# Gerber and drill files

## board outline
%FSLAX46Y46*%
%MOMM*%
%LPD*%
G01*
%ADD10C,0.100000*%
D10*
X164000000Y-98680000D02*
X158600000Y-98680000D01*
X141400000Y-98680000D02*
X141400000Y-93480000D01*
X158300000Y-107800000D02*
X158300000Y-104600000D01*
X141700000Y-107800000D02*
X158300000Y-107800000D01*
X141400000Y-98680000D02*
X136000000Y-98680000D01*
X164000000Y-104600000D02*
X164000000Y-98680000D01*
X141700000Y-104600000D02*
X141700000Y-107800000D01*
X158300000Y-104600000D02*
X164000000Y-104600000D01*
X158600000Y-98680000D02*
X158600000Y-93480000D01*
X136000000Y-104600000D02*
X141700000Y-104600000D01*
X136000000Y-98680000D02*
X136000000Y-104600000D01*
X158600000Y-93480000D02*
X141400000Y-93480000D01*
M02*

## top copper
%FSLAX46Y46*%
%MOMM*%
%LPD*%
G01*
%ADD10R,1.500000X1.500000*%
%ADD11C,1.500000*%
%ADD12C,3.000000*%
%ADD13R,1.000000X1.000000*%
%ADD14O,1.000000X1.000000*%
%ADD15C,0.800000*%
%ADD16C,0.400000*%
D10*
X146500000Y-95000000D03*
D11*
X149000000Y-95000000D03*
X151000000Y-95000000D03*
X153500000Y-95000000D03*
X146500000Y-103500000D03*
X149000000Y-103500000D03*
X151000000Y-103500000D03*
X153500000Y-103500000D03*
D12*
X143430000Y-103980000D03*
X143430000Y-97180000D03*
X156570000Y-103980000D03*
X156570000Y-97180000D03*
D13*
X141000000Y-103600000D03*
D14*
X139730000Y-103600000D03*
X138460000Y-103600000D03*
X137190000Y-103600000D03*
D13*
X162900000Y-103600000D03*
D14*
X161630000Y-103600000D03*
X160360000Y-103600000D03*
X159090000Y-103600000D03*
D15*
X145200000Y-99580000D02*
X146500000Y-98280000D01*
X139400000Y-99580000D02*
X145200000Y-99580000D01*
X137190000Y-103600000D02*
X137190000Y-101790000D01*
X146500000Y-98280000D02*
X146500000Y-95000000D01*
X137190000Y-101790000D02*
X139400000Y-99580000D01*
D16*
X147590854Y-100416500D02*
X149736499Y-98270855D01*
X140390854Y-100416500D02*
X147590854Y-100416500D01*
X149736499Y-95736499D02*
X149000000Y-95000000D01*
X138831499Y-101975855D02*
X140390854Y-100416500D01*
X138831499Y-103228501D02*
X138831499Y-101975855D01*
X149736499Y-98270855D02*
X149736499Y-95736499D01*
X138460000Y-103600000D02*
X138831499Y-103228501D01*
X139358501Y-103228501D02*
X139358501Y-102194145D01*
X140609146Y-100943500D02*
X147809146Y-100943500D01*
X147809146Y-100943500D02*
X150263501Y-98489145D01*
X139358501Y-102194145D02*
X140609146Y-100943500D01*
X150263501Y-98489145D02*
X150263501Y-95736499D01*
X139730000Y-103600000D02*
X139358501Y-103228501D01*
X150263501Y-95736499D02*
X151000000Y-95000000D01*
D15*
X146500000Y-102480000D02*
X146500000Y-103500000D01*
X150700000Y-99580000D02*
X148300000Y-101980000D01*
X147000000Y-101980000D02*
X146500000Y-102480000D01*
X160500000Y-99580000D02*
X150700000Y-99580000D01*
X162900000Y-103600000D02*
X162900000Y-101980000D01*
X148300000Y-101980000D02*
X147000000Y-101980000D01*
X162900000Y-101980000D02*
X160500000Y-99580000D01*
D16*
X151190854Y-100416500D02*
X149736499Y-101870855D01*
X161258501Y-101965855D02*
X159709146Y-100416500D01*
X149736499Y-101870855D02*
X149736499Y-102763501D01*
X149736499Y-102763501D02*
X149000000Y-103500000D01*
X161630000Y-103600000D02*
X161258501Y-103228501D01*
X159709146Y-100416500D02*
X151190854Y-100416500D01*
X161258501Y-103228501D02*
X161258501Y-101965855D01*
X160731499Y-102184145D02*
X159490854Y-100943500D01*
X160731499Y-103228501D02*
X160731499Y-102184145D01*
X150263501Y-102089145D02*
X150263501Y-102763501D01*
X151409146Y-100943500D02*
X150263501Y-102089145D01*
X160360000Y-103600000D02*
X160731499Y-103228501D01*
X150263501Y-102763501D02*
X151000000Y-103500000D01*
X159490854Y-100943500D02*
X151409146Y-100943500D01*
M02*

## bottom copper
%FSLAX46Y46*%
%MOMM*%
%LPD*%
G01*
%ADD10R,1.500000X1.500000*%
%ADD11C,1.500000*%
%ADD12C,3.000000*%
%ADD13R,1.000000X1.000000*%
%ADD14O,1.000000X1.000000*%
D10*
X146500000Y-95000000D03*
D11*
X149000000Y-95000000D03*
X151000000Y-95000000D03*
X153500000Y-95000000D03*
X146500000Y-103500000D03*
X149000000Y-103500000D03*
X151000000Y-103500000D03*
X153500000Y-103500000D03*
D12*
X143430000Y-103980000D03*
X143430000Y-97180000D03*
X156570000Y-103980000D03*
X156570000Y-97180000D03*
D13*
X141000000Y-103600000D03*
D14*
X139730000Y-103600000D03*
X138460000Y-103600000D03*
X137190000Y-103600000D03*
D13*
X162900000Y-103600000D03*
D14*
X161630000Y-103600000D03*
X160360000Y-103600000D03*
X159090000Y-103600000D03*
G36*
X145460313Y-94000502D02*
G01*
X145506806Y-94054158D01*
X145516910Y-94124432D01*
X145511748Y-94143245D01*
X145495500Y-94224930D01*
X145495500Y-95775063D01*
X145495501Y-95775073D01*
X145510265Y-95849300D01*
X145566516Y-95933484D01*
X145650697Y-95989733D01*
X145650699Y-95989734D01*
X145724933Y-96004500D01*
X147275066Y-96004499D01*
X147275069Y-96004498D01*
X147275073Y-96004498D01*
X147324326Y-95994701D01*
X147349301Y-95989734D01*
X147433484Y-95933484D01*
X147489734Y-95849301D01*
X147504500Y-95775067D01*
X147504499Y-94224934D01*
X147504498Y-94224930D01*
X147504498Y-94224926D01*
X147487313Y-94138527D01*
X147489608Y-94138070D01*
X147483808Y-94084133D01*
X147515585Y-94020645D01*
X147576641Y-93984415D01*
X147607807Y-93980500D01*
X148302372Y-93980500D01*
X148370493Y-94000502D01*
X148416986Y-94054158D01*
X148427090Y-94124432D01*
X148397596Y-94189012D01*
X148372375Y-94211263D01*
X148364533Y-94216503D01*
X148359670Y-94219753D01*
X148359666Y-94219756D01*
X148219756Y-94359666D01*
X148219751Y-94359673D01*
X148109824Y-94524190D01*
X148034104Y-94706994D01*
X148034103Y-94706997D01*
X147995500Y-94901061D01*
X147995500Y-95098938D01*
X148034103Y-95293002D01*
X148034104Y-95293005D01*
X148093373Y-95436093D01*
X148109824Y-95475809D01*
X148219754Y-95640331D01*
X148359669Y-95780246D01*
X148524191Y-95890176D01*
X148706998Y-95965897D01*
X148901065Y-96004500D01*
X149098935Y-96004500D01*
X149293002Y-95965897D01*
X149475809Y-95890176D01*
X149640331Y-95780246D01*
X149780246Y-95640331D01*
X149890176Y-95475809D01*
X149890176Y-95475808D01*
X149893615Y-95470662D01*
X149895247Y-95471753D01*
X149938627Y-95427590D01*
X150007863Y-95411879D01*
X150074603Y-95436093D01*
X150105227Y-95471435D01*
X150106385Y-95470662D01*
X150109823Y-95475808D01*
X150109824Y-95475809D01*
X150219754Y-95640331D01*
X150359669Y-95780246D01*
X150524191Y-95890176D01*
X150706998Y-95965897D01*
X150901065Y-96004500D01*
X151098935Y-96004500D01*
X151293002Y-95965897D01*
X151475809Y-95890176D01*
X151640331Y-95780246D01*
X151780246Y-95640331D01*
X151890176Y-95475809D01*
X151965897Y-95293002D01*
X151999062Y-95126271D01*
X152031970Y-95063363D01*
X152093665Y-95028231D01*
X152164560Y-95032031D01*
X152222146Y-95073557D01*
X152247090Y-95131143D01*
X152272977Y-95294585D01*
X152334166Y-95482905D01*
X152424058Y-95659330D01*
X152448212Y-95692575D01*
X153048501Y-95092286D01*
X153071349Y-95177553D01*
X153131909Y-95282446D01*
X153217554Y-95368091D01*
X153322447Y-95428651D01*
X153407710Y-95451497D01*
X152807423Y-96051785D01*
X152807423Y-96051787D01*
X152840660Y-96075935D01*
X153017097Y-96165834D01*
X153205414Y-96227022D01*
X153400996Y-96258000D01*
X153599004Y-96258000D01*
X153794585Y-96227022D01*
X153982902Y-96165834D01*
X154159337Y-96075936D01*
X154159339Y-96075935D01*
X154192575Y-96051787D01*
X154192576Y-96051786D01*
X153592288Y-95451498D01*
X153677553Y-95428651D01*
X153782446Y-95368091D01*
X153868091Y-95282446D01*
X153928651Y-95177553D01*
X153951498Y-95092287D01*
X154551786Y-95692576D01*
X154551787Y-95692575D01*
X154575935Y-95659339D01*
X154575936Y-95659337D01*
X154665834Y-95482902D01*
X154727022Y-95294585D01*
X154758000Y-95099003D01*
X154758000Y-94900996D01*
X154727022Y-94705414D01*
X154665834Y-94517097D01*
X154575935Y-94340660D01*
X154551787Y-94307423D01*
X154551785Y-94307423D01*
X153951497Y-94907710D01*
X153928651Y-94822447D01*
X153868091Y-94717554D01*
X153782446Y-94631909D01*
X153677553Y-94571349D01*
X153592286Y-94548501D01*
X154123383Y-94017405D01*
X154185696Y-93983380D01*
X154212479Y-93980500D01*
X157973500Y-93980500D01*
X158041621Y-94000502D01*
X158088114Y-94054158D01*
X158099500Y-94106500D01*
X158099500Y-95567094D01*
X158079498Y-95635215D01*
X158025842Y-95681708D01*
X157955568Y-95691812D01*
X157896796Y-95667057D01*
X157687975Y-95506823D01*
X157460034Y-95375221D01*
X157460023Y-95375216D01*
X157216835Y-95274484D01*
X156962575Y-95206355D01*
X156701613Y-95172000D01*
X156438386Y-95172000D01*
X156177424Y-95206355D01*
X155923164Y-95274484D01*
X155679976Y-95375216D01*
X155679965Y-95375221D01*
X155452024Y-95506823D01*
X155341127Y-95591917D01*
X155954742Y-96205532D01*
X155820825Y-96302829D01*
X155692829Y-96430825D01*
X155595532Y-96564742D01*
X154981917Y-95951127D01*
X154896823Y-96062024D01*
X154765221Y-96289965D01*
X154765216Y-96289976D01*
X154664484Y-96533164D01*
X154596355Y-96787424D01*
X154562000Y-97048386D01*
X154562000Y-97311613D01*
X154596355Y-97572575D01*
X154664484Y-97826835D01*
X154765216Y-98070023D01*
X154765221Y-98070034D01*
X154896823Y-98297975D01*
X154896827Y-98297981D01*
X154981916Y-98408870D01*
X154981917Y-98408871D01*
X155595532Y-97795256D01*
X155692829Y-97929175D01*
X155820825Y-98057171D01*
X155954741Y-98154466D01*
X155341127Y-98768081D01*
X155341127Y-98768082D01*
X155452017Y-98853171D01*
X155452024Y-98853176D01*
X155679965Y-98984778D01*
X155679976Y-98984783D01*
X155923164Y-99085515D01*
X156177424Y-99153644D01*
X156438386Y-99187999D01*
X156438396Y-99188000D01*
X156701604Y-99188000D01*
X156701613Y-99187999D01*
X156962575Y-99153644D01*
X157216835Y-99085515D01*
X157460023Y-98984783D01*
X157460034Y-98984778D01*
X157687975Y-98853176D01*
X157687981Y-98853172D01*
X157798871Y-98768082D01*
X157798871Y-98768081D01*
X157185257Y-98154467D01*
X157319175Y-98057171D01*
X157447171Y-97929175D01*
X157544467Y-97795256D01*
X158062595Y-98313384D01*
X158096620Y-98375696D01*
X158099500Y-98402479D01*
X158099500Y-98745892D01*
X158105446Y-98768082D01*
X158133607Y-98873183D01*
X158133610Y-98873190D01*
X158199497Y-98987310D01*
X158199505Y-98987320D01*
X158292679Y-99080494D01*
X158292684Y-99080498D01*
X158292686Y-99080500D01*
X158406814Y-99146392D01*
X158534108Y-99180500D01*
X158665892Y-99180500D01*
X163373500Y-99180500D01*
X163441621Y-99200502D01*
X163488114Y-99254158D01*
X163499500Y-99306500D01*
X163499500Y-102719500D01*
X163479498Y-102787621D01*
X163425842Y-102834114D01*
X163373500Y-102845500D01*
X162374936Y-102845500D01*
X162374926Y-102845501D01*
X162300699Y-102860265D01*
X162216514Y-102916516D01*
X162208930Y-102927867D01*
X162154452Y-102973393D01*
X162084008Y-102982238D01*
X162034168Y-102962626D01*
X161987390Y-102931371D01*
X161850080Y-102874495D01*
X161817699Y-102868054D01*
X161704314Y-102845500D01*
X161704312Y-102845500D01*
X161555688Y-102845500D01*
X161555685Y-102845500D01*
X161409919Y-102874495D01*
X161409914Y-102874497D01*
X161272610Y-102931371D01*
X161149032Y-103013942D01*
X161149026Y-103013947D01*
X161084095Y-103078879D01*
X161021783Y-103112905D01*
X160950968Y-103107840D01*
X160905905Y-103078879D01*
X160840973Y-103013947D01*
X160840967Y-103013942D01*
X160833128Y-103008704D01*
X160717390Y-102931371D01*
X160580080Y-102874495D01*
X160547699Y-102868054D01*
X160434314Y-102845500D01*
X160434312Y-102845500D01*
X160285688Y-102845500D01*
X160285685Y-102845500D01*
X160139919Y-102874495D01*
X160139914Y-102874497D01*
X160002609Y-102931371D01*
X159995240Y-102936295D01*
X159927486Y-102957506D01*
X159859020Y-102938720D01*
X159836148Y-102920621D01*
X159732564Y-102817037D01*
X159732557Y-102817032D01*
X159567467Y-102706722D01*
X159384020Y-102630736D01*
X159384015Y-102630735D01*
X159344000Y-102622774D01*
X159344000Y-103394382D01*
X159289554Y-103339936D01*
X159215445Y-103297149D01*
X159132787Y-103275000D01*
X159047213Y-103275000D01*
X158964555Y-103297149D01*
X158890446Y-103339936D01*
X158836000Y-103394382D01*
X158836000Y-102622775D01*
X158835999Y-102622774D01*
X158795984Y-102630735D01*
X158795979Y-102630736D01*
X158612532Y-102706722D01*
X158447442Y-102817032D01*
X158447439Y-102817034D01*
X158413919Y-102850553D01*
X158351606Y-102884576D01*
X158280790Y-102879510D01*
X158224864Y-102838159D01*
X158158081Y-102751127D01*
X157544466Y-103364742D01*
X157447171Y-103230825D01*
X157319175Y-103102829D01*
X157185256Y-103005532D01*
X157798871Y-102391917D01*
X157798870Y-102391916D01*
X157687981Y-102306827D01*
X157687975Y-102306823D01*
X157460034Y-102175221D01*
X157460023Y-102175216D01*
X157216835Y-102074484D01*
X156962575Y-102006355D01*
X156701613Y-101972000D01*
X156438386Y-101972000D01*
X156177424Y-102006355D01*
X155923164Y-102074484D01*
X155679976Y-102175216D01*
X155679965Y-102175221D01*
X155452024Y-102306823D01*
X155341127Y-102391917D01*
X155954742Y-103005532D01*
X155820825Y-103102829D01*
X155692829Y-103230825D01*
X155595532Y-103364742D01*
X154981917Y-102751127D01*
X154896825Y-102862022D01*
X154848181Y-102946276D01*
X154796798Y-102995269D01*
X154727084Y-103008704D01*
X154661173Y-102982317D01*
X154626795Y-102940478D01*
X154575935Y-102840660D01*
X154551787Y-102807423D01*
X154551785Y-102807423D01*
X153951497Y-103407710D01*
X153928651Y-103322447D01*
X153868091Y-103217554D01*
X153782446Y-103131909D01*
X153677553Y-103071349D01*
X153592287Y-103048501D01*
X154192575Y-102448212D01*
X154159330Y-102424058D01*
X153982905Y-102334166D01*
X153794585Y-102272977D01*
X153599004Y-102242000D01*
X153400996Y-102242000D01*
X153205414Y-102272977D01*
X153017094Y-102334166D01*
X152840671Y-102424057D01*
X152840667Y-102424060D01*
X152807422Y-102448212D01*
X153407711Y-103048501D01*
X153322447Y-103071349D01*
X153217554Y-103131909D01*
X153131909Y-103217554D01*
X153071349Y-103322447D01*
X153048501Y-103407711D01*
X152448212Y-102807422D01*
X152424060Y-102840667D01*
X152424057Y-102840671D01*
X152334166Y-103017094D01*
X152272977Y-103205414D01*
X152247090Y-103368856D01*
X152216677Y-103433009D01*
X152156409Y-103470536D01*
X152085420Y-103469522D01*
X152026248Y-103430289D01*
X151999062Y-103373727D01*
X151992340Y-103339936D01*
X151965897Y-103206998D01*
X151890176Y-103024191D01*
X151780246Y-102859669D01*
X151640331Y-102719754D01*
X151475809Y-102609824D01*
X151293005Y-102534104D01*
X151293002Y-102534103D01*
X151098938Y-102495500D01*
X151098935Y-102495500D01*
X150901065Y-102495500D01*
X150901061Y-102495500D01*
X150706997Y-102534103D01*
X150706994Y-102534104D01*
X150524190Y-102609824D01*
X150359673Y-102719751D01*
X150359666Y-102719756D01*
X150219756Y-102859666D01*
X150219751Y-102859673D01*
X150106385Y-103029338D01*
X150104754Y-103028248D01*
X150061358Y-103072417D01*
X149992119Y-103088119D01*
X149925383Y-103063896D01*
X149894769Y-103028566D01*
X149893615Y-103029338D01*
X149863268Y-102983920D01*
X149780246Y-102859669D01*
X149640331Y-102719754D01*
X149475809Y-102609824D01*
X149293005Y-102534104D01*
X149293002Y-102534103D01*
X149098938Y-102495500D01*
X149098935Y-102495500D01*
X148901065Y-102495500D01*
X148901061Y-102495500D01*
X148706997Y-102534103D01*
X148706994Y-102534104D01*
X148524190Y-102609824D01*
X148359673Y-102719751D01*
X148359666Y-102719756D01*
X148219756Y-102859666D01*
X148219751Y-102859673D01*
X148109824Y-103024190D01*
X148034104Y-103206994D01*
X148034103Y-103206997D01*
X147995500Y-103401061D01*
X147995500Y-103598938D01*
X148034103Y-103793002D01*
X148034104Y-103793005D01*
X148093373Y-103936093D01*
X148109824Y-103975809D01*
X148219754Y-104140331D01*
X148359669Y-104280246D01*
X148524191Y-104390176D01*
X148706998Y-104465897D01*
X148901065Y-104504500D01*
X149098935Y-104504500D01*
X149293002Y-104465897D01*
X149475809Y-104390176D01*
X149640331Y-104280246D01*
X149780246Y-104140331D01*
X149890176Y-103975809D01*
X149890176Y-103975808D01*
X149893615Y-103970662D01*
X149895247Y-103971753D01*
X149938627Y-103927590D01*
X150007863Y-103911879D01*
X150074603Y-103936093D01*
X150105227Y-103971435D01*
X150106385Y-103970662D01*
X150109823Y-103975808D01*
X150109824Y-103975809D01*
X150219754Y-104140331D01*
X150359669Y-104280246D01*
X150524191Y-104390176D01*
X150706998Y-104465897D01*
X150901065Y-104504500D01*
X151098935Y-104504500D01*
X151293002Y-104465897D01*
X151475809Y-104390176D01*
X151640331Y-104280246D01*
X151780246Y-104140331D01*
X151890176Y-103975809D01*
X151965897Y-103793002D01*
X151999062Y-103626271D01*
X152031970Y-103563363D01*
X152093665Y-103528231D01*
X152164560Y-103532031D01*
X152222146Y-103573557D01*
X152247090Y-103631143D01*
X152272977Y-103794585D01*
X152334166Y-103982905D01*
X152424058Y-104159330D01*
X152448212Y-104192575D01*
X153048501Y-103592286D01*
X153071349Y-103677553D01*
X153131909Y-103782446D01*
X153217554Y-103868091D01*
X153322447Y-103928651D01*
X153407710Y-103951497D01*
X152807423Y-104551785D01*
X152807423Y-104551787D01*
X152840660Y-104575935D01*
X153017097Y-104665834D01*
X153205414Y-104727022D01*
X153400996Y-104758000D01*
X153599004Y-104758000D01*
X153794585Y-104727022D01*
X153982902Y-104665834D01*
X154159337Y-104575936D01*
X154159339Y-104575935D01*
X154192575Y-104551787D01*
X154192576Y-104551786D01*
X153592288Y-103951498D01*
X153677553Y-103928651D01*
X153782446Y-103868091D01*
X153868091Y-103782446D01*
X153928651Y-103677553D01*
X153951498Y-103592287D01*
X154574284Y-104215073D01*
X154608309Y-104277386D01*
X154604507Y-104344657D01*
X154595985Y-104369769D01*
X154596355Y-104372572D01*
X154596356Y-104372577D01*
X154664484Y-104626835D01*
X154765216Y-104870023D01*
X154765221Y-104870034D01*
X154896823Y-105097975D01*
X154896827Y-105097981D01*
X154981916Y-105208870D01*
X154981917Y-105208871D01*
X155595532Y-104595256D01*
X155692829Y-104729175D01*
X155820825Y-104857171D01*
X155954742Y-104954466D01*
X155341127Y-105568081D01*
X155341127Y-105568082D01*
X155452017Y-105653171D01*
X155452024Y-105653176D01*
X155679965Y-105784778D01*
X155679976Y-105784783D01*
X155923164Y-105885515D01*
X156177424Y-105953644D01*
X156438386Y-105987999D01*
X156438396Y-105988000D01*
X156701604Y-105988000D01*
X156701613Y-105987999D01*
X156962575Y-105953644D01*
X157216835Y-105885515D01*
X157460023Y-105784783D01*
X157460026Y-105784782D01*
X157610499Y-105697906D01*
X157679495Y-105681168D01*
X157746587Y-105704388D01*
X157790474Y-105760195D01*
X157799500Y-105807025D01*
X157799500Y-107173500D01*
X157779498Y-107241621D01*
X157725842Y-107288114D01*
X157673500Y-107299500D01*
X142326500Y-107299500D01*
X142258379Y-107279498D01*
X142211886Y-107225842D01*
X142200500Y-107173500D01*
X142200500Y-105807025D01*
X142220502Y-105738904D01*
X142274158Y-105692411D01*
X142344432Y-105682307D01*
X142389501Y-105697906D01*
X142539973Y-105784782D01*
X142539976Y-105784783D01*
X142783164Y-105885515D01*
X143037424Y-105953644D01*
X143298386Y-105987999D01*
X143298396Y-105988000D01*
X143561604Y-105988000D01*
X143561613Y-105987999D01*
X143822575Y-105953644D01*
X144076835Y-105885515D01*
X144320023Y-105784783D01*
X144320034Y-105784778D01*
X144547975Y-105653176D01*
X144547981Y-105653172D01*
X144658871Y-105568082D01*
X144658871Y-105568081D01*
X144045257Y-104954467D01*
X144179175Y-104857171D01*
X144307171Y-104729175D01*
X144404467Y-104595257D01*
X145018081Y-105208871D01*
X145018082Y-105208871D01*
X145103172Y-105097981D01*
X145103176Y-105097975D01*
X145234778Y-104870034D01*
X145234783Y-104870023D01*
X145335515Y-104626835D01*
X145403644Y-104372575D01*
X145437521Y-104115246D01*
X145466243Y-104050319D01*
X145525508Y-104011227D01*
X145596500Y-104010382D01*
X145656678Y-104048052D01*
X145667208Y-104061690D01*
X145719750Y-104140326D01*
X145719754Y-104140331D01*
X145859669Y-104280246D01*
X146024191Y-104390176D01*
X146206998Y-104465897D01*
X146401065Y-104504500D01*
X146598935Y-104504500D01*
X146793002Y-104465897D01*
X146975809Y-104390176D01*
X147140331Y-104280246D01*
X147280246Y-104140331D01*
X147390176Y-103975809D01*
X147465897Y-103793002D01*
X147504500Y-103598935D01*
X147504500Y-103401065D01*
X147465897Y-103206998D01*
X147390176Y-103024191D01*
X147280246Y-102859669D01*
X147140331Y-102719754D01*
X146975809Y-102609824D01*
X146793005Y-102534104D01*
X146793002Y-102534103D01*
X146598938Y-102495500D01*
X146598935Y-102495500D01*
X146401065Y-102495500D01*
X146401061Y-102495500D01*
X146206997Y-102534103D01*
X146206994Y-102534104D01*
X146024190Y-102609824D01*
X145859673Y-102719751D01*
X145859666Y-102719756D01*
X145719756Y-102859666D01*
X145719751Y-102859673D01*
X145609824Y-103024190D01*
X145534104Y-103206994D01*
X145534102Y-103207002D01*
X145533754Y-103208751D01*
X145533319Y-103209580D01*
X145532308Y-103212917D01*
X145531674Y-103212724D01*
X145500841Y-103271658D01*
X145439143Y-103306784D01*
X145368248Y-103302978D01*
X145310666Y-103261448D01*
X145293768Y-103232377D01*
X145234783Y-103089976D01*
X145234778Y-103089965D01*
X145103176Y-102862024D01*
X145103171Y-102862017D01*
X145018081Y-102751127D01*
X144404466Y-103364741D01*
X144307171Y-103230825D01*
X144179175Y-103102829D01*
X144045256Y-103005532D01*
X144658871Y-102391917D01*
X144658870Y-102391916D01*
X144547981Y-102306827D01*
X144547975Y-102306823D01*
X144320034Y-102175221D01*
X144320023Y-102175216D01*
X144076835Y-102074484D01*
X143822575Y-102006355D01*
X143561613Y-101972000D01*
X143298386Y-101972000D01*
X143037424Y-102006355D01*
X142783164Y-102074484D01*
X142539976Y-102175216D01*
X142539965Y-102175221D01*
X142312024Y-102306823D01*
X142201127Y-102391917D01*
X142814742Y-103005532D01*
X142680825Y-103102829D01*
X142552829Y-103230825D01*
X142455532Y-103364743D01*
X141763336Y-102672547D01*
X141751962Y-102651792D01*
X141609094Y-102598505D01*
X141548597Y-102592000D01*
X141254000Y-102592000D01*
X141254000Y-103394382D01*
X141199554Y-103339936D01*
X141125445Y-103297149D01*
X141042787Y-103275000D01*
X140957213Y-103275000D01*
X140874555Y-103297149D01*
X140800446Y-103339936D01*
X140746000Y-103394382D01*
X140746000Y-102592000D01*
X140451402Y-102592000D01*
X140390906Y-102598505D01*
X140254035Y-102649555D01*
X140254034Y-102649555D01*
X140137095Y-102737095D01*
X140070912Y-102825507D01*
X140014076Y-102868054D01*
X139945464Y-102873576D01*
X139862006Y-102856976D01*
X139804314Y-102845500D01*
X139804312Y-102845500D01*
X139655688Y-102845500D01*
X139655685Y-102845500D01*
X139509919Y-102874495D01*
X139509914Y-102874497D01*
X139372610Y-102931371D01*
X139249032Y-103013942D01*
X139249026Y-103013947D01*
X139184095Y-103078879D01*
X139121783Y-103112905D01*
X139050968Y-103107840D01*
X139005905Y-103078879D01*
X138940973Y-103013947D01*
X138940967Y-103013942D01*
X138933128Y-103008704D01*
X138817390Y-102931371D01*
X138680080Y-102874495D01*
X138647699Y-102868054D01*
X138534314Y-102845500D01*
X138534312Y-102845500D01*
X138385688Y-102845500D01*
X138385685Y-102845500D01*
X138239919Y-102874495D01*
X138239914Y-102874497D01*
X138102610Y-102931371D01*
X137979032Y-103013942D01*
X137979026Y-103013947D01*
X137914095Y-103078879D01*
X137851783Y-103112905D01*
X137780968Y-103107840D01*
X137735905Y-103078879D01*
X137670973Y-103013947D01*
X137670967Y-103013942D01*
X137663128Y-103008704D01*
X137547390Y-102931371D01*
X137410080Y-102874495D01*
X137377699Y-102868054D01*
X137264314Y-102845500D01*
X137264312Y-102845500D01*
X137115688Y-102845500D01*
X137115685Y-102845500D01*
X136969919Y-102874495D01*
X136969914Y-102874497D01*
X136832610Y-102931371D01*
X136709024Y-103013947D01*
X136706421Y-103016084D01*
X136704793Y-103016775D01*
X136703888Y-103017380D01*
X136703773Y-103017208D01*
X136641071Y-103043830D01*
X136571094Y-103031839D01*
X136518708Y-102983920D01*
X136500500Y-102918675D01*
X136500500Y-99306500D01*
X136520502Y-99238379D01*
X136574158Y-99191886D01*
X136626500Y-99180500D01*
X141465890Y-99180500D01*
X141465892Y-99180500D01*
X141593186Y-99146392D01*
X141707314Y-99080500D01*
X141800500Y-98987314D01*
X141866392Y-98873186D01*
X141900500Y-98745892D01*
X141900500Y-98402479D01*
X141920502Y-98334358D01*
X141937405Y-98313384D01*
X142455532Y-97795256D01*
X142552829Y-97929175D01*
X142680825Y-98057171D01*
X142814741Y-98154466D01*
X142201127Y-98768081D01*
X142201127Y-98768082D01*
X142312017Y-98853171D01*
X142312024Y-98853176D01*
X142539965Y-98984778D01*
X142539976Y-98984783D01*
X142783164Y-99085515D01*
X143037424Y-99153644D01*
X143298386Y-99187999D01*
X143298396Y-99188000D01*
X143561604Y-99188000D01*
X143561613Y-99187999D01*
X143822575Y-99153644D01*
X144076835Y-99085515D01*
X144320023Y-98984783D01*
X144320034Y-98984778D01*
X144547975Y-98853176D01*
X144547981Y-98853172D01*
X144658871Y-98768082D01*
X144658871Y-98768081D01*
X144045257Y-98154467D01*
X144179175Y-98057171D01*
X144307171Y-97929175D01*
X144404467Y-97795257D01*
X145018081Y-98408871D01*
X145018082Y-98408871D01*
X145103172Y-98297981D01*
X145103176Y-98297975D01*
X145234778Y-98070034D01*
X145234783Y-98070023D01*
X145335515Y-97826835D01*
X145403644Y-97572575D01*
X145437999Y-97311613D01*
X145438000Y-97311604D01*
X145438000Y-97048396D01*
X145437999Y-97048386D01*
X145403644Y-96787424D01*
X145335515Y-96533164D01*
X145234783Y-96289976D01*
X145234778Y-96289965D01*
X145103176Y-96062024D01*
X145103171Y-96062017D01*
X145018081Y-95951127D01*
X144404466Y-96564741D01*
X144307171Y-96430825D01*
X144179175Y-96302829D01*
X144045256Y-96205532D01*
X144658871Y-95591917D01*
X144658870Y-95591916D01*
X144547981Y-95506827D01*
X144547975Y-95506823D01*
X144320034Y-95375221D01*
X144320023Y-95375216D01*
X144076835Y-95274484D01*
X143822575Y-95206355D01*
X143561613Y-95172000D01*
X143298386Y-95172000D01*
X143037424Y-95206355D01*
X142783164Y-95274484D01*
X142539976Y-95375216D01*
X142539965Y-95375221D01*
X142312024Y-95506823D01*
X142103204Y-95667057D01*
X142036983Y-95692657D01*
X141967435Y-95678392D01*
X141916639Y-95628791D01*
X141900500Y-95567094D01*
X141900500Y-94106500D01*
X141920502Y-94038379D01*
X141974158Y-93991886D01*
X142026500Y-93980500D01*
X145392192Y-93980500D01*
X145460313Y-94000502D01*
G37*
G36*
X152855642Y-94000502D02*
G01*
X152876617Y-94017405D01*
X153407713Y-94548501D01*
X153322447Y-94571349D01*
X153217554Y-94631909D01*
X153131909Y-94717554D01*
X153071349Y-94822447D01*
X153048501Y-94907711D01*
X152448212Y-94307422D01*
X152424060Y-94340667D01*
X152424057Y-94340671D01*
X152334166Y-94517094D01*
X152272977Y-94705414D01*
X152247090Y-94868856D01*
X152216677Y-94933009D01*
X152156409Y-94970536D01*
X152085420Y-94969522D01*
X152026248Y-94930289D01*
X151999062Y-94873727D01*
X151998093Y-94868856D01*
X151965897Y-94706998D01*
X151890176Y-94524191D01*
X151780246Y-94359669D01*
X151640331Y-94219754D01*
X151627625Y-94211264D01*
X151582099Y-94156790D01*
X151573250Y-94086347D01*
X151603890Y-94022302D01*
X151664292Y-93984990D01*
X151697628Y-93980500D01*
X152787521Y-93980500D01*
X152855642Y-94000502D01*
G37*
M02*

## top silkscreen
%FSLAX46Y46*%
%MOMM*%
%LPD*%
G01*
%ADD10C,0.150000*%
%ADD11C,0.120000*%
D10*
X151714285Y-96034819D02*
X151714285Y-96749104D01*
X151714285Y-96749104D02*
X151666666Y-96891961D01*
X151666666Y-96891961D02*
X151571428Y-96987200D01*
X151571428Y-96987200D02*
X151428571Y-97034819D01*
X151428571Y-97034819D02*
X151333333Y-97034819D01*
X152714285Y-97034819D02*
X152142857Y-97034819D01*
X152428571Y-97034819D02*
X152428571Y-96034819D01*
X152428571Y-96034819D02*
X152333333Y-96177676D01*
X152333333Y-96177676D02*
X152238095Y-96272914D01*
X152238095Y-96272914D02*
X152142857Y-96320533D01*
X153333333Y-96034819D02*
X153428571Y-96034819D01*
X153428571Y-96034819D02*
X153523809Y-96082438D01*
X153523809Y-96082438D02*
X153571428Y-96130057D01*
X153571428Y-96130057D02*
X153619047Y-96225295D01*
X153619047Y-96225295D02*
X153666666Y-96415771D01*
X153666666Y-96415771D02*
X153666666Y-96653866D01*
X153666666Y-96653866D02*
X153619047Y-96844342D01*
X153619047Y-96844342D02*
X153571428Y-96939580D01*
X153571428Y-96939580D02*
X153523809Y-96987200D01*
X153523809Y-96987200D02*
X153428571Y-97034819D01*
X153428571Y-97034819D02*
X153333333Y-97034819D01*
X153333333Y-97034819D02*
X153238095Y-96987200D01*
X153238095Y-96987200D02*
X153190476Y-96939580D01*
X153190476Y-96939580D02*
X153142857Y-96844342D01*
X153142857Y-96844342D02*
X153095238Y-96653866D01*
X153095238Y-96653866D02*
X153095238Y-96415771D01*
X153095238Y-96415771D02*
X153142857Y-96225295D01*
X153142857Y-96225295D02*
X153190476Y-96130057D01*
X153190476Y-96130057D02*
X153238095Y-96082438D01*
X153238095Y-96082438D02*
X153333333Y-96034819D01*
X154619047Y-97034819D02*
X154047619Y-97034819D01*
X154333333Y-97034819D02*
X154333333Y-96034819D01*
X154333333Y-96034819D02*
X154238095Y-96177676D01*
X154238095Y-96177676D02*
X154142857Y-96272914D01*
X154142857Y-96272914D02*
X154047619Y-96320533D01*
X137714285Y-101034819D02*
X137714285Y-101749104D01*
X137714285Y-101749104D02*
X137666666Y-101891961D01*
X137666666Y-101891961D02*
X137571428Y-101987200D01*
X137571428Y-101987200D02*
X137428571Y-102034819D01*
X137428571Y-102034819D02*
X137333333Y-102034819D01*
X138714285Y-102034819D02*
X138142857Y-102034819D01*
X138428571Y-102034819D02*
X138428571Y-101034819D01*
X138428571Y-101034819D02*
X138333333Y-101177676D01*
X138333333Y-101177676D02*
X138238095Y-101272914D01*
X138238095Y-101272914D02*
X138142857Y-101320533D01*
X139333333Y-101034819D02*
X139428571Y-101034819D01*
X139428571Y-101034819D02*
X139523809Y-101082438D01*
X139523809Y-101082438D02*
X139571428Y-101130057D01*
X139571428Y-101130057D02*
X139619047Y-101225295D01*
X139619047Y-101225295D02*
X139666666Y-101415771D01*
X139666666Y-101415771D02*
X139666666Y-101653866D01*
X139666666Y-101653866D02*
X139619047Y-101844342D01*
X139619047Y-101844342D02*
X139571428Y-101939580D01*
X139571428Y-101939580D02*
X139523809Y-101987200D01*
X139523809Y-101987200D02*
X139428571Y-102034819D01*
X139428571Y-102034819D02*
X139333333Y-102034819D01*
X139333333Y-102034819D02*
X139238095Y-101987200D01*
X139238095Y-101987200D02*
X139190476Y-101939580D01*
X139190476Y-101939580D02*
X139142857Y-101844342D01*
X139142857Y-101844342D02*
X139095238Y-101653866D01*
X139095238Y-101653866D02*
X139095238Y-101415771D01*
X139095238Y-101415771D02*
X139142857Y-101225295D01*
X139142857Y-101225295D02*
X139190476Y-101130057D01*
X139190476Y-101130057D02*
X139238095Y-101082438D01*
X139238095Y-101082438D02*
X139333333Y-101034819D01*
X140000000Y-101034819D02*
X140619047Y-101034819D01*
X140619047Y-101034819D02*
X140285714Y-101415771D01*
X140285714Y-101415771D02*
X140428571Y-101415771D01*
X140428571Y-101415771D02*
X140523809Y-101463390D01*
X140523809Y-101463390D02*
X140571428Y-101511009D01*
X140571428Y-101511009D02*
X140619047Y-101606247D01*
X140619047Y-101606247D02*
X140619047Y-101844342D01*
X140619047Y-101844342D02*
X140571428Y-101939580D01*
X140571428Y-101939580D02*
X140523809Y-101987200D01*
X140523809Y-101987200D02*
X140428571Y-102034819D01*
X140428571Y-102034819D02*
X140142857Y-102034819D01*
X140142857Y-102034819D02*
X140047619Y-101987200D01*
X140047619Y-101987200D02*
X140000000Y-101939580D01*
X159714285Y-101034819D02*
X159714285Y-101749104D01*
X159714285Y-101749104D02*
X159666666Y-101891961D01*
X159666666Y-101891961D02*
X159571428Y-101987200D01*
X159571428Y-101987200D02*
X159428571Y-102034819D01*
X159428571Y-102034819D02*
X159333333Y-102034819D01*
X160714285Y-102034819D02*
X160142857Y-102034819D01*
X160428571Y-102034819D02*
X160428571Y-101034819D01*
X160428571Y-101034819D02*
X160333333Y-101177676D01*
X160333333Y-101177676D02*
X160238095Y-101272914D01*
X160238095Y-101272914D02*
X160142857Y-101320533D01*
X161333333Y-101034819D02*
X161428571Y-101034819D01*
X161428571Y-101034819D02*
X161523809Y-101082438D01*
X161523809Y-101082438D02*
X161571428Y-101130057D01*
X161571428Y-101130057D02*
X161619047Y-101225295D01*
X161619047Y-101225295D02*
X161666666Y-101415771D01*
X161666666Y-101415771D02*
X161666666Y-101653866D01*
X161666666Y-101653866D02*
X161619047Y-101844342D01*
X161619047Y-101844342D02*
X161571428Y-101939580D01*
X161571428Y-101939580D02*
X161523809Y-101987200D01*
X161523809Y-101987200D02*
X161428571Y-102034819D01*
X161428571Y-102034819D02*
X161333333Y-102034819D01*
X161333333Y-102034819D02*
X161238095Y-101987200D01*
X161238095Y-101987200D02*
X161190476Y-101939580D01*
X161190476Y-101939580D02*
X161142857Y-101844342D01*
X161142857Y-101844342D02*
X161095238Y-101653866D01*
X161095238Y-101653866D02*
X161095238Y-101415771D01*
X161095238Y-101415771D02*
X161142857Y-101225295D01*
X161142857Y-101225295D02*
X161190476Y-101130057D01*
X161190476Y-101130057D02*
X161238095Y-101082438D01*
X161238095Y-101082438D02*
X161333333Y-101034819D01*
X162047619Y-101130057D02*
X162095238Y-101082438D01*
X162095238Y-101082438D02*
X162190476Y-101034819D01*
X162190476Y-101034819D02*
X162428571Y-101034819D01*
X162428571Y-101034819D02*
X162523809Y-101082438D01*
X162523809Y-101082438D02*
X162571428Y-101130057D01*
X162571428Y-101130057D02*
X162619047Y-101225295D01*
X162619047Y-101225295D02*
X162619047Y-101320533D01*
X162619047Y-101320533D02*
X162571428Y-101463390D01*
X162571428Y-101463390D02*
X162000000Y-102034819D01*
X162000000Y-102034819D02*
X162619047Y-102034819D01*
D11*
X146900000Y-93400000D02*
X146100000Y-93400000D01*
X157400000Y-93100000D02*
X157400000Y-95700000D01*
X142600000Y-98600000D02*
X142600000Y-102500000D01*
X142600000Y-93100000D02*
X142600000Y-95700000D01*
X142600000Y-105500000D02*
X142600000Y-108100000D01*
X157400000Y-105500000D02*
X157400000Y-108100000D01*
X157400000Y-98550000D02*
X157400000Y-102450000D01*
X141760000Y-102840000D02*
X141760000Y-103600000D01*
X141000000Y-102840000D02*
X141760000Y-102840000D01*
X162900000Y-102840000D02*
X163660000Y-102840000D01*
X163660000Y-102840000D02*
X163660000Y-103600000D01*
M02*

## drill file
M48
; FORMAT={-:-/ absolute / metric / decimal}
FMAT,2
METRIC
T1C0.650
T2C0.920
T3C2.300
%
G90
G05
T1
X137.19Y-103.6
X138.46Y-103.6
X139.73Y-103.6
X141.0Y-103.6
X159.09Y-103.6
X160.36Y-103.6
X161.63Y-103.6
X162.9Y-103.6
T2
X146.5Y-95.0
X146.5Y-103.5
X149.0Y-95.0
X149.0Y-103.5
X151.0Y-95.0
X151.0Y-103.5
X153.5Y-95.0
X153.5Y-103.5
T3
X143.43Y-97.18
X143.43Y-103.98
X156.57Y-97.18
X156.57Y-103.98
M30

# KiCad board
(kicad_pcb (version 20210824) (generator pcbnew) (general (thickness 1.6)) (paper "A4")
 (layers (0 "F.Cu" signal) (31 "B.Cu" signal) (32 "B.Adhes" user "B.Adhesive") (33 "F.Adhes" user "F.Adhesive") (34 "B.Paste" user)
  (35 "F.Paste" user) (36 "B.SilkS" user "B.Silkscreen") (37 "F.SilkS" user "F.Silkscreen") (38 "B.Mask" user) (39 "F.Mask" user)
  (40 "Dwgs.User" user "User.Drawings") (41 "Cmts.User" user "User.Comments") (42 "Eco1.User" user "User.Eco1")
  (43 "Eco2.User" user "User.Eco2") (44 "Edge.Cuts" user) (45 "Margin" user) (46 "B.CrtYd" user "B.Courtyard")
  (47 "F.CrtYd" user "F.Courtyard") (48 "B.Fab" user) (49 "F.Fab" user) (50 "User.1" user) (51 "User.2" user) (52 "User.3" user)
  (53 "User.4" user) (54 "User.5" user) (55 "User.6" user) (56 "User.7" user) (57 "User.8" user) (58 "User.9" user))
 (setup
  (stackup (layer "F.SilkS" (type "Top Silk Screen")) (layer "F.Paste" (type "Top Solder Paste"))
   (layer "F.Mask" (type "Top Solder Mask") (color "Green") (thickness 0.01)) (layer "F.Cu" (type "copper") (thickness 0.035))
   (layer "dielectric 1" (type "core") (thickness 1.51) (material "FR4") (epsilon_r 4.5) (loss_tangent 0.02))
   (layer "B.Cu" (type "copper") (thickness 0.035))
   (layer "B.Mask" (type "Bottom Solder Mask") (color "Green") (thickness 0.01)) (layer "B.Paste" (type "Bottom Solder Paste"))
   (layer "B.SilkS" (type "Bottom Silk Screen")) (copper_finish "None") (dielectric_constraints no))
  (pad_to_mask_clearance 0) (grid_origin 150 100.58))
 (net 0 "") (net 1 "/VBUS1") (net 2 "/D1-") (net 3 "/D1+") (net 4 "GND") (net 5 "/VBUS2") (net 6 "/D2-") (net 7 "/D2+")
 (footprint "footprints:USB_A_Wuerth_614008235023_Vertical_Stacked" (layer "F.Cu") (at 150 95)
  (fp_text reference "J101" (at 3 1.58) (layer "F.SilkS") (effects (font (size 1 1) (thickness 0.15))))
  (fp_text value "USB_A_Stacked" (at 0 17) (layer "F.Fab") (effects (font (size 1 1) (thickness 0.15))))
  (fp_line (start -3.1 -1.6) (end -3.9 -1.6) (layer "F.SilkS") (width 0.12))
  (fp_line (start 7.4 -1.9) (end 7.4 0.7) (layer "F.SilkS") (width 0.12))
  (fp_line (start -7.4 3.6) (end -7.4 7.5) (layer "F.SilkS") (width 0.12))
  (fp_line (start -7.4 -1.9) (end -7.4 0.7) (layer "F.SilkS") (width 0.12))
  (fp_line (start -7.4 10.5) (end -7.4 13.1) (layer "F.SilkS") (width 0.12))
  (fp_line (start 7.4 10.5) (end 7.4 13.1) (layer "F.SilkS") (width 0.12))
  (fp_line (start 7.4 3.55) (end 7.4 7.45) (layer "F.SilkS") (width 0.12))
  (pad "1" thru_hole rect locked (at -3.5 0) (size 1.5 1.5) (drill 0.92) (layers *.Cu *.Mask) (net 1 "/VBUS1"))
  (pad "2" thru_hole circle locked (at -1 0) (size 1.5 1.5) (drill 0.92) (layers *.Cu *.Mask) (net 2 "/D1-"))
  (pad "3" thru_hole circle locked (at 1 0) (size 1.5 1.5) (drill 0.92) (layers *.Cu *.Mask) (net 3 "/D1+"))
  (pad "4" thru_hole circle locked (at 3.5 0) (size 1.5 1.5) (drill 0.92) (layers *.Cu *.Mask) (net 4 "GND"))
  (pad "5" thru_hole circle locked (at -3.5 8.5) (size 1.5 1.5) (drill 0.92) (layers *.Cu *.Mask) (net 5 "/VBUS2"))
  (pad "6" thru_hole circle locked (at -1 8.5) (size 1.5 1.5) (drill 0.92) (layers *.Cu *.Mask) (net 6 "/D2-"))
  (pad "7" thru_hole circle locked (at 1 8.5) (size 1.5 1.5) (drill 0.92) (layers *.Cu *.Mask) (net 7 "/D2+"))
  (pad "8" thru_hole circle locked (at 3.5 8.5) (size 1.5 1.5) (drill 0.92) (layers *.Cu *.Mask) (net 4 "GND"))
  (pad "9" thru_hole circle locked (at -6.57 8.98) (size 3 3) (drill 2.3) (layers *.Cu *.Mask) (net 4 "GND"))
  (pad "9" thru_hole circle locked (at -6.57 2.18) (size 3 3) (drill 2.3) (layers *.Cu *.Mask) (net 4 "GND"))
  (pad "9" thru_hole circle locked (at 6.57 8.98) (size 3 3) (drill 2.3) (layers *.Cu *.Mask) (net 4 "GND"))
  (pad "9" thru_hole circle locked (at 6.57 2.18) (size 3 3) (drill 2.3) (layers *.Cu *.Mask) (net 4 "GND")))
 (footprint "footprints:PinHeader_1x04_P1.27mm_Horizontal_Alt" (layer "F.Cu") (at 141 103.6 -90)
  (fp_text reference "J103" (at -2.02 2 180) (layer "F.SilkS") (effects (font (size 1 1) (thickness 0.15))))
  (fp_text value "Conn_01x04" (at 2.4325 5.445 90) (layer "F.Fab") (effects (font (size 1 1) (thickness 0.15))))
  (fp_line (start -0.76 -0.76) (end 0 -0.76) (layer "F.SilkS") (width 0.12))
  (fp_line (start -0.76 0) (end -0.76 -0.76) (layer "F.SilkS") (width 0.12))
  (pad "1" thru_hole rect locked (at 0 0 270) (size 1 1) (drill 0.65) (layers *.Cu *.Mask) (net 4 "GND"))
  (pad "2" thru_hole oval locked (at 0 1.27 270) (size 1 1) (drill 0.65) (layers *.Cu *.Mask) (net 3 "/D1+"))
  (pad "3" thru_hole oval locked (at 0 2.54 270) (size 1 1) (drill 0.65) (layers *.Cu *.Mask) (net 2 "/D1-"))
  (pad "4" thru_hole oval locked (at 0 3.81 270) (size 1 1) (drill 0.65) (layers *.Cu *.Mask) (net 1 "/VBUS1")))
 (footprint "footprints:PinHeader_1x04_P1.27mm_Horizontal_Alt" (layer "F.Cu") (at 162.9 103.6 -90)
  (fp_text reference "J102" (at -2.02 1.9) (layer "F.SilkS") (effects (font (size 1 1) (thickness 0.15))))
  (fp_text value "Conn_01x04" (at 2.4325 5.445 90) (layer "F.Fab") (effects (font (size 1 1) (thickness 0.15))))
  (fp_line (start -0.76 0) (end -0.76 -0.76) (layer "F.SilkS") (width 0.12))
  (fp_line (start -0.76 -0.76) (end 0 -0.76) (layer "F.SilkS") (width 0.12))
  (pad "1" thru_hole rect locked (at 0 0 270) (size 1 1) (drill 0.65) (layers *.Cu *.Mask) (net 5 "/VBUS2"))
  (pad "2" thru_hole oval locked (at 0 1.27 270) (size 1 1) (drill 0.65) (layers *.Cu *.Mask) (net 6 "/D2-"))
  (pad "3" thru_hole oval locked (at 0 2.54 270) (size 1 1) (drill 0.65) (layers *.Cu *.Mask) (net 7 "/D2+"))
  (pad "4" thru_hole oval locked (at 0 3.81 270) (size 1 1) (drill 0.65) (layers *.Cu *.Mask) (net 4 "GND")))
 (gr_line (start 164 98.68) (end 158.6 98.68) (layer "Edge.Cuts") (width 0.1))
 (gr_line (start 141.4 98.68) (end 141.4 93.48) (layer "Edge.Cuts") (width 0.1))
 (gr_line (start 158.3 107.8) (end 158.3 104.6) (layer "Edge.Cuts") (width 0.1))
 (gr_line (start 141.7 107.8) (end 158.3 107.8) (layer "Edge.Cuts") (width 0.1))
 (gr_line (start 141.4 98.68) (end 136 98.68) (layer "Edge.Cuts") (width 0.1))
 (gr_line (start 164 104.6) (end 164 98.68) (layer "Edge.Cuts") (width 0.1))
 (gr_line (start 141.7 104.6) (end 141.7 107.8) (layer "Edge.Cuts") (width 0.1))
 (gr_line (start 158.3 104.6) (end 164 104.6) (layer "Edge.Cuts") (width 0.1))
 (gr_line (start 158.6 98.68) (end 158.6 93.48) (layer "Edge.Cuts") (width 0.1))
 (gr_line (start 136 104.6) (end 141.7 104.6) (layer "Edge.Cuts") (width 0.1))
 (gr_line (start 136 98.68) (end 136 104.6) (layer "Edge.Cuts") (width 0.1))
 (gr_line (start 158.6 93.48) (end 141.4 93.48) (layer "Edge.Cuts") (width 0.1))
 (segment (start 145.2 99.58) (end 146.5 98.28) (width 0.8) (layer "F.Cu") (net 1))
 (segment (start 139.4 99.58) (end 145.2 99.58) (width 0.8) (layer "F.Cu") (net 1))
 (segment (start 137.19 103.6) (end 137.19 101.79) (width 0.8) (layer "F.Cu") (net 1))
 (segment (start 146.5 98.28) (end 146.5 95) (width 0.8) (layer "F.Cu") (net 1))
 (segment (start 137.19 101.79) (end 139.4 99.58) (width 0.8) (layer "F.Cu") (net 1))
 (segment (start 147.590854 100.4165) (end 149.736499 98.270855) (width 0.4) (layer "F.Cu") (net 2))
 (segment (start 140.390854 100.4165) (end 147.590854 100.4165) (width 0.4) (layer "F.Cu") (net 2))
 (segment (start 149.736499 95.736499) (end 149 95) (width 0.4) (layer "F.Cu") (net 2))
 (segment (start 138.831499 101.975855) (end 140.390854 100.4165) (width 0.4) (layer "F.Cu") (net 2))
 (segment (start 138.831499 103.228501) (end 138.831499 101.975855) (width 0.4) (layer "F.Cu") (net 2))
 (segment (start 149.736499 98.270855) (end 149.736499 95.736499) (width 0.4) (layer "F.Cu") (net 2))
 (segment (start 138.46 103.6) (end 138.831499 103.228501) (width 0.4) (layer "F.Cu") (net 2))
 (segment (start 139.358501 103.228501) (end 139.358501 102.194145) (width 0.4) (layer "F.Cu") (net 3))
 (segment (start 140.609146 100.9435) (end 147.809146 100.9435) (width 0.4) (layer "F.Cu") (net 3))
 (segment (start 147.809146 100.9435) (end 150.263501 98.489145) (width 0.4) (layer "F.Cu") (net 3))
 (segment (start 139.358501 102.194145) (end 140.609146 100.9435) (width 0.4) (layer "F.Cu") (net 3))
 (segment (start 150.263501 98.489145) (end 150.263501 95.736499) (width 0.4) (layer "F.Cu") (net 3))
 (segment (start 139.73 103.6) (end 139.358501 103.228501) (width 0.4) (layer "F.Cu") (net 3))
 (segment (start 150.263501 95.736499) (end 151 95) (width 0.4) (layer "F.Cu") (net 3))
 (segment (start 146.5 102.48) (end 146.5 103.5) (width 0.8) (layer "F.Cu") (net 5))
 (segment (start 150.7 99.58) (end 148.3 101.98) (width 0.8) (layer "F.Cu") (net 5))
 (segment (start 147 101.98) (end 146.5 102.48) (width 0.8) (layer "F.Cu") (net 5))
 (segment (start 160.5 99.58) (end 150.7 99.58) (width 0.8) (layer "F.Cu") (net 5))
 (segment (start 162.9 103.6) (end 162.9 101.98) (width 0.8) (layer "F.Cu") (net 5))
 (segment (start 148.3 101.98) (end 147 101.98) (width 0.8) (layer "F.Cu") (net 5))
 (segment (start 162.9 101.98) (end 160.5 99.58) (width 0.8) (layer "F.Cu") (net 5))
 (segment (start 151.190854 100.4165) (end 149.736499 101.870855) (width 0.4) (layer "F.Cu") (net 6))
 (segment (start 161.258501 101.965855) (end 159.709146 100.4165) (width 0.4) (layer "F.Cu") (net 6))
 (segment (start 149.736499 101.870855) (end 149.736499 102.763501) (width 0.4) (layer "F.Cu") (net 6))
 (segment (start 149.736499 102.763501) (end 149 103.5) (width 0.4) (layer "F.Cu") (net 6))
 (segment (start 161.63 103.6) (end 161.258501 103.228501) (width 0.4) (layer "F.Cu") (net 6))
 (segment (start 159.709146 100.4165) (end 151.190854 100.4165) (width 0.4) (layer "F.Cu") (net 6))
 (segment (start 161.258501 103.228501) (end 161.258501 101.965855) (width 0.4) (layer "F.Cu") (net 6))
 (segment (start 160.731499 102.184145) (end 159.490854 100.9435) (width 0.4) (layer "F.Cu") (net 7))
 (segment (start 160.731499 103.228501) (end 160.731499 102.184145) (width 0.4) (layer "F.Cu") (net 7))
 (segment (start 150.263501 102.089145) (end 150.263501 102.763501) (width 0.4) (layer "F.Cu") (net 7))
 (segment (start 151.409146 100.9435) (end 150.263501 102.089145) (width 0.4) (layer "F.Cu") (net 7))
 (segment (start 160.36 103.6) (end 160.731499 103.228501) (width 0.4) (layer "F.Cu") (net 7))
 (segment (start 150.263501 102.763501) (end 151 103.5) (width 0.4) (layer "F.Cu") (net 7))
 (segment (start 159.490854 100.9435) (end 151.409146 100.9435) (width 0.4) (layer "F.Cu") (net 7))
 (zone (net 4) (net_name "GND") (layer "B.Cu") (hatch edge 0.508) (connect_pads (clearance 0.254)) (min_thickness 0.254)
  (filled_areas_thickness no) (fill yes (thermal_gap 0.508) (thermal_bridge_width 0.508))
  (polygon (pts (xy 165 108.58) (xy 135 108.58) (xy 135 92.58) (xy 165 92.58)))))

